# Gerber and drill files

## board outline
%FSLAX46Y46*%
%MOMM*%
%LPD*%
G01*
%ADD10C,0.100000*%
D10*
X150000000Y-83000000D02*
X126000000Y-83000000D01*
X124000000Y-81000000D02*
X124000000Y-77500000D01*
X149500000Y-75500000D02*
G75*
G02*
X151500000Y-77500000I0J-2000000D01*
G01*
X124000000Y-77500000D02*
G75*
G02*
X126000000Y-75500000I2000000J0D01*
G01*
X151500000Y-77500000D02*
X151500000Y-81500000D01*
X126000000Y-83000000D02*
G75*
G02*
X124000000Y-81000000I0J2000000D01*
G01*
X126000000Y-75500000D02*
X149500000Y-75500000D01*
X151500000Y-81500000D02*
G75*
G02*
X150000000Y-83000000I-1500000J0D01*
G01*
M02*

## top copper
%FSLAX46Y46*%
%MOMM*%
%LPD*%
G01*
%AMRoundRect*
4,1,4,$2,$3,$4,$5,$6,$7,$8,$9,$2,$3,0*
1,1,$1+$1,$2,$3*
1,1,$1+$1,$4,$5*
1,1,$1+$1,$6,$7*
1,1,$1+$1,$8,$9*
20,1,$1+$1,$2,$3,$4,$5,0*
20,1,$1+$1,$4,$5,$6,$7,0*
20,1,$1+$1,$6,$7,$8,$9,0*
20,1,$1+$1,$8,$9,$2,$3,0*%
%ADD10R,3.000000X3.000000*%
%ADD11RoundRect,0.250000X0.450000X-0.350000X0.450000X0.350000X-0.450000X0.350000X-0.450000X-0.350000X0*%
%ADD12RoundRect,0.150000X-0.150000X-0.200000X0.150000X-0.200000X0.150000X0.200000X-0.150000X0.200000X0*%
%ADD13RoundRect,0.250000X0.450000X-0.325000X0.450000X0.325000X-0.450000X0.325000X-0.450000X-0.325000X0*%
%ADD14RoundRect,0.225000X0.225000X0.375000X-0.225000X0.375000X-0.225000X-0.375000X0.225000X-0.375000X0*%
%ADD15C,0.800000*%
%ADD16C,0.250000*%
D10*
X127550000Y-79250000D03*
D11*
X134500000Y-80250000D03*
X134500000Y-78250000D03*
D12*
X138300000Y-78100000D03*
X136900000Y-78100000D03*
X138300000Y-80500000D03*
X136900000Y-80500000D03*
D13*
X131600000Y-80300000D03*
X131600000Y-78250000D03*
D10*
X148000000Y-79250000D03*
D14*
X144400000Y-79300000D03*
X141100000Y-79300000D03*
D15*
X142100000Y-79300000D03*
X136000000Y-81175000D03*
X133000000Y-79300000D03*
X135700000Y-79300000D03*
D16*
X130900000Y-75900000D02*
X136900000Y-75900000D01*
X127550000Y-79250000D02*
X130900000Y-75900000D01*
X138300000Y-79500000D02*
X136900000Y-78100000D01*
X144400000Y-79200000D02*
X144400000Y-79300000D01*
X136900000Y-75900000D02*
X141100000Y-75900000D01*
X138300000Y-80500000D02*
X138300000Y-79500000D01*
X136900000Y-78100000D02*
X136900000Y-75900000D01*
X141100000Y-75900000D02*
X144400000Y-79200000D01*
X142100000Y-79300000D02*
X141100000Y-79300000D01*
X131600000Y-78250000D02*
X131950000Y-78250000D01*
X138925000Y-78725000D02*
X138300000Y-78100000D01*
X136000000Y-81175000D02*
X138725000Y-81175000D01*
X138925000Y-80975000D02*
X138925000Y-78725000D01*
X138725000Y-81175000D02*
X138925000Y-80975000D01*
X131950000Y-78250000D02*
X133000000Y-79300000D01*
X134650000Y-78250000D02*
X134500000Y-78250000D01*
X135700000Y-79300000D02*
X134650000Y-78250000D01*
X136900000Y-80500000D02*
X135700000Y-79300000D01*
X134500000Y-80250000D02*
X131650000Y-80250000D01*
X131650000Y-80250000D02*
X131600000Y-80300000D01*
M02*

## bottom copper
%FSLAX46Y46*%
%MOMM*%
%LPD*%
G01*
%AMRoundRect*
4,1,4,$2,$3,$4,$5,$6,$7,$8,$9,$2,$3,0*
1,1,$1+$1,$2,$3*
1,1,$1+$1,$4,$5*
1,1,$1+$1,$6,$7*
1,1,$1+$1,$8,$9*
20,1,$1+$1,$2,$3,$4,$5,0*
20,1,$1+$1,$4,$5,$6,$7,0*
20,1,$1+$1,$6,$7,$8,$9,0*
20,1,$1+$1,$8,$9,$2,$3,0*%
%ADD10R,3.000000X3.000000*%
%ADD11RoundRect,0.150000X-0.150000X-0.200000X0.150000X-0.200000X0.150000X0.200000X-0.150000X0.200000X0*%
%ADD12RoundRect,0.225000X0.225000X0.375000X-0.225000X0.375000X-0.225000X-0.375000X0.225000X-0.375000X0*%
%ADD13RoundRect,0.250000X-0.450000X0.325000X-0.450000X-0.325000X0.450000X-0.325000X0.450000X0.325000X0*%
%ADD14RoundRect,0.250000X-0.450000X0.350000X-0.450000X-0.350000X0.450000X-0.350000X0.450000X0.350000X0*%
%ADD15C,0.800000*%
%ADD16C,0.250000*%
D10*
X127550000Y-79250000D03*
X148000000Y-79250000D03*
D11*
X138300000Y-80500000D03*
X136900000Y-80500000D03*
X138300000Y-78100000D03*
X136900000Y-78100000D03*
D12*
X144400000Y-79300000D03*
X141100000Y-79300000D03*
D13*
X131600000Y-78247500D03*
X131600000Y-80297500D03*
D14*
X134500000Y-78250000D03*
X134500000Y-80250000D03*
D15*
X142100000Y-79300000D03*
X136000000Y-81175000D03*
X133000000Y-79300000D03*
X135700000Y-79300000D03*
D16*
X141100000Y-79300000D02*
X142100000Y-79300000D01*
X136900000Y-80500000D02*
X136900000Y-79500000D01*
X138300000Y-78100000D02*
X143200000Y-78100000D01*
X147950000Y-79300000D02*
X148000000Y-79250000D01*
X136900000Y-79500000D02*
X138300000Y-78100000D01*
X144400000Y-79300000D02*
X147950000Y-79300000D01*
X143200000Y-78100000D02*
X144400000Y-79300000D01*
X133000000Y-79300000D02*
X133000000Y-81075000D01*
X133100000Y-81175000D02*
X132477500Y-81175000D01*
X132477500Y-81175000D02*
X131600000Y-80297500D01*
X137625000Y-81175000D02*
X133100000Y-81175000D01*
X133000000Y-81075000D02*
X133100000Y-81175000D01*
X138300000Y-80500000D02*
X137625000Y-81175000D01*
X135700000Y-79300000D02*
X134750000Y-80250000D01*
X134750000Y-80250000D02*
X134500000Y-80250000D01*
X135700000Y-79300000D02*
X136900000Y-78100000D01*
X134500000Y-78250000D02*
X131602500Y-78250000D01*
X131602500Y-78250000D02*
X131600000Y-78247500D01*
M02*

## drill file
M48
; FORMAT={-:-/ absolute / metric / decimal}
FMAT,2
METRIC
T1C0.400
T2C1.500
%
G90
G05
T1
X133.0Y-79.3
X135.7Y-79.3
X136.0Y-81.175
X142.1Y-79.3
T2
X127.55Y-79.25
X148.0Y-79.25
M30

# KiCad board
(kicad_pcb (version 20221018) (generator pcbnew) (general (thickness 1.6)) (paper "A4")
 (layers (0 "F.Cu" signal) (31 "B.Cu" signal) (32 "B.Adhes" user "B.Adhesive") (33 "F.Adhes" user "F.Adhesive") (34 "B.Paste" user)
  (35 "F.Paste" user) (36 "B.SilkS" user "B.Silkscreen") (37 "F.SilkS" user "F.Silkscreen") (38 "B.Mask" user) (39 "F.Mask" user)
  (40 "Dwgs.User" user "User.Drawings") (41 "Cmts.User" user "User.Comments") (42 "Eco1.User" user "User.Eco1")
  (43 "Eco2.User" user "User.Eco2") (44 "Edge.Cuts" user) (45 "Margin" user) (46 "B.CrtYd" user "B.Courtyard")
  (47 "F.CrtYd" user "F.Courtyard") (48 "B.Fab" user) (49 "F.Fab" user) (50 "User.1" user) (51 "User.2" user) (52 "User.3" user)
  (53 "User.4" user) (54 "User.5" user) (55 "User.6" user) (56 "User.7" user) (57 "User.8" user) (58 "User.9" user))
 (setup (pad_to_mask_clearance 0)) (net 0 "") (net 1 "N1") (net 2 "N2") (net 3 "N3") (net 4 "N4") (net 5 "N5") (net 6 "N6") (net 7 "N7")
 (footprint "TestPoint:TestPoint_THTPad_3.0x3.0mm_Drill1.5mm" (layer "F.Cu") (at 127.55 79.25)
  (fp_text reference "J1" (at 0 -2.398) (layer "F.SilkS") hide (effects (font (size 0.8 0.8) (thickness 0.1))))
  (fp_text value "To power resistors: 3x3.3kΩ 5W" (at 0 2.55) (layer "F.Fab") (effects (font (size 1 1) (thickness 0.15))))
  (pad "1" thru_hole rect (at 0 0) (size 3 3) (drill 1.5) (layers "*.Cu" "*.Mask") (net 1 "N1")))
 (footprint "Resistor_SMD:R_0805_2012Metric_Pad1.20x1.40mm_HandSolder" (layer "F.Cu") (at 134.5 79.25 90)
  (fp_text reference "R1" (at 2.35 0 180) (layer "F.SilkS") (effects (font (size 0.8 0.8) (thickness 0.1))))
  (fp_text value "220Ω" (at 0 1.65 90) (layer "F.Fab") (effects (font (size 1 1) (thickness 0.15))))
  (pad "1" smd roundrect (at -1 0 90) (size 1.2 1.4) (layers "F.Cu" "F.Paste" "F.Mask") (roundrect_rratio 0.2083333333) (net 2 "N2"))
  (pad "2" smd roundrect (at 1 0 90) (size 1.2 1.4) (layers "F.Cu" "F.Paste" "F.Mask") (roundrect_rratio 0.2083333333) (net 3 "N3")))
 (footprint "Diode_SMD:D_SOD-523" (layer "F.Cu") (at 137.6 78.1 180)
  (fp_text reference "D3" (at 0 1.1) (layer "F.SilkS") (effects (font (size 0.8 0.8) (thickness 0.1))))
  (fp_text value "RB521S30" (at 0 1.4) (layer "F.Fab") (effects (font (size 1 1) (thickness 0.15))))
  (pad "1" smd roundrect (at -0.7 0) (size 0.6 0.7) (layers "F.Cu" "F.Paste" "F.Mask") (roundrect_rratio 0.25) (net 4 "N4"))
  (pad "2" smd roundrect (at 0.7 0) (size 0.6 0.7) (layers "F.Cu" "F.Paste" "F.Mask") (roundrect_rratio 0.25) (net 1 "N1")))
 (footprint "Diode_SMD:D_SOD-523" (layer "F.Cu") (at 137.6 80.5 180)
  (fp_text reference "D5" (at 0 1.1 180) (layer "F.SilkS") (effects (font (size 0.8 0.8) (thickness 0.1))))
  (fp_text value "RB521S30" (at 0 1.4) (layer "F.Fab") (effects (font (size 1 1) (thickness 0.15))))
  (pad "1" smd roundrect (at -0.7 0) (size 0.6 0.7) (layers "F.Cu" "F.Paste" "F.Mask") (roundrect_rratio 0.25) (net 1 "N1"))
  (pad "2" smd roundrect (at 0.7 0) (size 0.6 0.7) (layers "F.Cu" "F.Paste" "F.Mask") (roundrect_rratio 0.25) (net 3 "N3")))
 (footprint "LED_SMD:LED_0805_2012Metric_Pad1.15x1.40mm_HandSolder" (layer "F.Cu") (at 131.6 79.275 90)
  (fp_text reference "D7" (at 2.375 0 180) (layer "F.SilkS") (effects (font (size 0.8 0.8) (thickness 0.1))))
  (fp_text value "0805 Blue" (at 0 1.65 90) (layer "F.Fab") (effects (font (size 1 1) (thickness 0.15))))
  (pad "1" smd roundrect (at -1.025 0 90) (size 1.15 1.4) (layers "F.Cu" "F.Paste" "F.Mask") (roundrect_rratio 0.2173913043) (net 2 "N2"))
  (pad "2" smd roundrect (at 1.025 0 90) (size 1.15 1.4) (layers "F.Cu" "F.Paste" "F.Mask") (roundrect_rratio 0.2173913043) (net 4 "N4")))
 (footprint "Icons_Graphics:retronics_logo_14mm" (layer "F.Cu") (at 131.3 82)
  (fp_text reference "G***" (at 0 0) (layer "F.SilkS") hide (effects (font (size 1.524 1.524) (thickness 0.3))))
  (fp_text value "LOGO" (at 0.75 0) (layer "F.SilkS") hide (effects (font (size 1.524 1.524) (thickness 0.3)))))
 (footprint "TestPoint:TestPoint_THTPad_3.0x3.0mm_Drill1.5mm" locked (layer "F.Cu") (at 148 79.25)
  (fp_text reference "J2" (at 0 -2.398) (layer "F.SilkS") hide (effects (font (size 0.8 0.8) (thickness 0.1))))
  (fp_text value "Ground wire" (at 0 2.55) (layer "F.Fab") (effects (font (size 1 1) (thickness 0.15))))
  (pad "1" thru_hole rect locked (at 0 0) (size 3 3) (drill 1.5) (layers "*.Cu" "*.Mask") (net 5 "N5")))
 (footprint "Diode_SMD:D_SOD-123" (layer "F.Cu") (at 142.75 79.3 180)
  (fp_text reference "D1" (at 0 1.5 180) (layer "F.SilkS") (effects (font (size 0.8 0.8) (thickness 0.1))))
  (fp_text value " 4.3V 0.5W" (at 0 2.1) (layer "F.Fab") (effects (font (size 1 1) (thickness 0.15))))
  (pad "1" smd roundrect (at -1.65 0 180) (size 0.9 1.2) (layers "F.Cu" "F.Paste" "F.Mask") (roundrect_rratio 0.25) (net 1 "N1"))
  (pad "2" smd roundrect (at 1.65 0 180) (size 0.9 1.2) (layers "F.Cu" "F.Paste" "F.Mask") (roundrect_rratio 0.25) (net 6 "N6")))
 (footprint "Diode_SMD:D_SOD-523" (layer "B.Cu") (at 137.6 80.5 180)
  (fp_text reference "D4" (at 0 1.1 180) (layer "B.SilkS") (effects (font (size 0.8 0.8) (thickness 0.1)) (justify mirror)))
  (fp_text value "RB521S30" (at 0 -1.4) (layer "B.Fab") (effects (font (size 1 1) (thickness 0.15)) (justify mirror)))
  (pad "1" smd roundrect (at -0.7 0) (size 0.6 0.7) (layers "B.Cu" "B.Paste" "B.Mask") (roundrect_rratio 0.25) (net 4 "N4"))
  (pad "2" smd roundrect (at 0.7 0) (size 0.6 0.7) (layers "B.Cu" "B.Paste" "B.Mask") (roundrect_rratio 0.25) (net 5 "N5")))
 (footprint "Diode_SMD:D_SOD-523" (layer "B.Cu") (at 137.6 78.1 180)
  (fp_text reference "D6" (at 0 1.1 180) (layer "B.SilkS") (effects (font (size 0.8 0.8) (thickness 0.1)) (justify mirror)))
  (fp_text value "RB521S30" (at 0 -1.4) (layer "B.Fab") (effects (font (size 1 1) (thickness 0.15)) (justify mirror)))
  (pad "1" smd roundrect (at -0.7 0) (size 0.6 0.7) (layers "B.Cu" "B.Paste" "B.Mask") (roundrect_rratio 0.25) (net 5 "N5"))
  (pad "2" smd roundrect (at 0.7 0) (size 0.6 0.7) (layers "B.Cu" "B.Paste" "B.Mask") (roundrect_rratio 0.25) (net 3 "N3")))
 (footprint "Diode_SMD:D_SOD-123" (layer "B.Cu") (at 142.75 79.3 180)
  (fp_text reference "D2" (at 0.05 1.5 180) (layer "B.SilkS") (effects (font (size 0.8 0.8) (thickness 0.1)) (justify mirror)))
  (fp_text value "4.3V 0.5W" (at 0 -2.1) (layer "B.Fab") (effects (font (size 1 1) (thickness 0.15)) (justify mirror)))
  (pad "1" smd roundrect (at -1.65 0 180) (size 0.9 1.2) (layers "B.Cu" "B.Paste" "B.Mask") (roundrect_rratio 0.25) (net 5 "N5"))
  (pad "2" smd roundrect (at 1.65 0 180) (size 0.9 1.2) (layers "B.Cu" "B.Paste" "B.Mask") (roundrect_rratio 0.25) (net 6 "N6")))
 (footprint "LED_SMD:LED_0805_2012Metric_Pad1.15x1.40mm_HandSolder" (layer "B.Cu") (at 131.6 79.2725 -90)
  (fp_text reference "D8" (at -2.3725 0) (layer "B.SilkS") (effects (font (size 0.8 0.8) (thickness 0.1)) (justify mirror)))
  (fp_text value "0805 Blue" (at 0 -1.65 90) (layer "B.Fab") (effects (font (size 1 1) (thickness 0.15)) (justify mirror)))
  (pad "1" smd roundrect (at -1.025 0 270) (size 1.15 1.4) (layers "B.Cu" "B.Paste" "B.Mask") (roundrect_rratio 0.2173913043) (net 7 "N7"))
  (pad "2" smd roundrect (at 1.025 0 270) (size 1.15 1.4) (layers "B.Cu" "B.Paste" "B.Mask") (roundrect_rratio 0.2173913043) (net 4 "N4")))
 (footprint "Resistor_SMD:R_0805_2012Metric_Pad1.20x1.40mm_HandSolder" (layer "B.Cu") (at 134.5 79.25 -90)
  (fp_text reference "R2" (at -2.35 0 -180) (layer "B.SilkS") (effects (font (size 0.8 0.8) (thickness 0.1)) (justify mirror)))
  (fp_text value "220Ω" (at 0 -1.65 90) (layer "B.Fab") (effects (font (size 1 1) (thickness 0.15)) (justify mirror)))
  (pad "1" smd roundrect (at -1 0 270) (size 1.2 1.4) (layers "B.Cu" "B.Paste" "B.Mask") (roundrect_rratio 0.2083333333) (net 7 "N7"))
  (pad "2" smd roundrect (at 1 0 270) (size 1.2 1.4) (layers "B.Cu" "B.Paste" "B.Mask") (roundrect_rratio 0.2083333333) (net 3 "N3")))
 (gr_line (start 150 83) (end 126 83) (stroke (width 0.1) (type default)) (layer "Edge.Cuts"))
 (gr_line (start 124 81) (end 124 77.5) (stroke (width 0.1) (type default)) (layer "Edge.Cuts"))
 (gr_arc (start 149.5 75.5) (mid 150.914214 76.085786) (end 151.5 77.5) (stroke (width 0.1) (type default)) (layer "Edge.Cuts"))
 (gr_arc (start 124 77.5) (mid 124.585786 76.085786) (end 126 75.5) (stroke (width 0.1) (type default)) (layer "Edge.Cuts"))
 (gr_line (start 151.5 77.5) (end 151.5 81.5) (stroke (width 0.1) (type default)) (layer "Edge.Cuts"))
 (gr_arc (start 126 83) (mid 124.585786 82.414214) (end 124 81) (stroke (width 0.1) (type default)) (layer "Edge.Cuts"))
 (gr_line (start 126 75.5) (end 149.5 75.5) (stroke (width 0.1) (type default)) (layer "Edge.Cuts"))
 (gr_arc (start 151.5 81.5) (mid 151.06066 82.56066) (end 150 83) (stroke (width 0.1) (type default)) (layer "Edge.Cuts"))
 (segment (start 130.9 75.9) (end 136.9 75.9) (width 0.25) (layer "F.Cu") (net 1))
 (segment (start 127.55 79.25) (end 130.9 75.9) (width 0.25) (layer "F.Cu") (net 1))
 (segment (start 138.3 79.5) (end 136.9 78.1) (width 0.25) (layer "F.Cu") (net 1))
 (segment (start 144.4 79.2) (end 144.4 79.3) (width 0.25) (layer "F.Cu") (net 1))
 (segment (start 136.9 75.9) (end 141.1 75.9) (width 0.25) (layer "F.Cu") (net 1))
 (segment (start 138.3 80.5) (end 138.3 79.5) (width 0.25) (layer "F.Cu") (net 1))
 (segment (start 136.9 78.1) (end 136.9 75.9) (width 0.25) (layer "F.Cu") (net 1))
 (segment (start 141.1 75.9) (end 144.4 79.2) (width 0.25) (layer "F.Cu") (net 1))
 (segment (start 142.1 79.3) (end 141.1 79.3) (width 0.25) (layer "F.Cu") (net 6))
 (via (at 142.1 79.3) (size 0.8) (drill 0.4) (layers "F.Cu" "B.Cu") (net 6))
 (segment (start 141.1 79.3) (end 142.1 79.3) (width 0.25) (layer "B.Cu") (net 6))
 (segment (start 136.9 80.5) (end 136.9 79.5) (width 0.25) (layer "B.Cu") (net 5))
 (segment (start 138.3 78.1) (end 143.2 78.1) (width 0.25) (layer "B.Cu") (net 5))
 (segment (start 147.95 79.3) (end 148 79.25) (width 0.25) (layer "B.Cu") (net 5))
 (segment (start 136.9 79.5) (end 138.3 78.1) (width 0.25) (layer "B.Cu") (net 5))
 (segment (start 144.4 79.3) (end 147.95 79.3) (width 0.25) (layer "B.Cu") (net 5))
 (segment (start 143.2 78.1) (end 144.4 79.3) (width 0.25) (layer "B.Cu") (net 5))
 (segment (start 131.6 78.25) (end 131.95 78.25) (width 0.25) (layer "F.Cu") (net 4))
 (segment (start 138.925 78.725) (end 138.3 78.1) (width 0.25) (layer "F.Cu") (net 4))
 (segment (start 136 81.175) (end 138.725 81.175) (width 0.25) (layer "F.Cu") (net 4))
 (segment (start 138.925 80.975) (end 138.925 78.725) (width 0.25) (layer "F.Cu") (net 4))
 (segment (start 138.725 81.175) (end 138.925 80.975) (width 0.25) (layer "F.Cu") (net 4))
 (segment (start 131.95 78.25) (end 133 79.3) (width 0.25) (layer "F.Cu") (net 4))
 (via (at 136 81.175) (size 0.8) (drill 0.4) (layers "F.Cu" "B.Cu") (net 4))
 (via (at 133 79.3) (size 0.8) (drill 0.4) (layers "F.Cu" "B.Cu") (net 4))
 (segment (start 133 79.3) (end 133 81.075) (width 0.25) (layer "B.Cu") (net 4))
 (segment (start 133.1 81.175) (end 132.4775 81.175) (width 0.25) (layer "B.Cu") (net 4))
 (segment (start 132.4775 81.175) (end 131.6 80.2975) (width 0.25) (layer "B.Cu") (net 4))
 (segment (start 137.625 81.175) (end 133.1 81.175) (width 0.25) (layer "B.Cu") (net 4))
 (segment (start 133 81.075) (end 133.1 81.175) (width 0.25) (layer "B.Cu") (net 4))
 (segment (start 138.3 80.5) (end 137.625 81.175) (width 0.25) (layer "B.Cu") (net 4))
 (segment (start 134.65 78.25) (end 134.5 78.25) (width 0.25) (layer "F.Cu") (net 3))
 (segment (start 135.7 79.3) (end 134.65 78.25) (width 0.25) (layer "F.Cu") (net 3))
 (segment (start 136.9 80.5) (end 135.7 79.3) (width 0.25) (layer "F.Cu") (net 3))
 (via (at 135.7 79.3) (size 0.8) (drill 0.4) (layers "F.Cu" "B.Cu") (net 3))
 (segment (start 135.7 79.3) (end 134.75 80.25) (width 0.25) (layer "B.Cu") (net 3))
 (segment (start 134.75 80.25) (end 134.5 80.25) (width 0.25) (layer "B.Cu") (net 3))
 (segment (start 135.7 79.3) (end 136.9 78.1) (width 0.25) (layer "B.Cu") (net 3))
 (segment (start 134.5 80.25) (end 131.65 80.25) (width 0.25) (layer "F.Cu") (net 2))
 (segment (start 131.65 80.25) (end 131.6 80.3) (width 0.25) (layer "F.Cu") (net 2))
 (segment (start 134.5 78.25) (end 131.6025 78.25) (width 0.25) (layer "B.Cu") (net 7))
 (segment (start 131.6025 78.25) (end 131.6 78.2475) (width 0.25) (layer "B.Cu") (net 7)))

